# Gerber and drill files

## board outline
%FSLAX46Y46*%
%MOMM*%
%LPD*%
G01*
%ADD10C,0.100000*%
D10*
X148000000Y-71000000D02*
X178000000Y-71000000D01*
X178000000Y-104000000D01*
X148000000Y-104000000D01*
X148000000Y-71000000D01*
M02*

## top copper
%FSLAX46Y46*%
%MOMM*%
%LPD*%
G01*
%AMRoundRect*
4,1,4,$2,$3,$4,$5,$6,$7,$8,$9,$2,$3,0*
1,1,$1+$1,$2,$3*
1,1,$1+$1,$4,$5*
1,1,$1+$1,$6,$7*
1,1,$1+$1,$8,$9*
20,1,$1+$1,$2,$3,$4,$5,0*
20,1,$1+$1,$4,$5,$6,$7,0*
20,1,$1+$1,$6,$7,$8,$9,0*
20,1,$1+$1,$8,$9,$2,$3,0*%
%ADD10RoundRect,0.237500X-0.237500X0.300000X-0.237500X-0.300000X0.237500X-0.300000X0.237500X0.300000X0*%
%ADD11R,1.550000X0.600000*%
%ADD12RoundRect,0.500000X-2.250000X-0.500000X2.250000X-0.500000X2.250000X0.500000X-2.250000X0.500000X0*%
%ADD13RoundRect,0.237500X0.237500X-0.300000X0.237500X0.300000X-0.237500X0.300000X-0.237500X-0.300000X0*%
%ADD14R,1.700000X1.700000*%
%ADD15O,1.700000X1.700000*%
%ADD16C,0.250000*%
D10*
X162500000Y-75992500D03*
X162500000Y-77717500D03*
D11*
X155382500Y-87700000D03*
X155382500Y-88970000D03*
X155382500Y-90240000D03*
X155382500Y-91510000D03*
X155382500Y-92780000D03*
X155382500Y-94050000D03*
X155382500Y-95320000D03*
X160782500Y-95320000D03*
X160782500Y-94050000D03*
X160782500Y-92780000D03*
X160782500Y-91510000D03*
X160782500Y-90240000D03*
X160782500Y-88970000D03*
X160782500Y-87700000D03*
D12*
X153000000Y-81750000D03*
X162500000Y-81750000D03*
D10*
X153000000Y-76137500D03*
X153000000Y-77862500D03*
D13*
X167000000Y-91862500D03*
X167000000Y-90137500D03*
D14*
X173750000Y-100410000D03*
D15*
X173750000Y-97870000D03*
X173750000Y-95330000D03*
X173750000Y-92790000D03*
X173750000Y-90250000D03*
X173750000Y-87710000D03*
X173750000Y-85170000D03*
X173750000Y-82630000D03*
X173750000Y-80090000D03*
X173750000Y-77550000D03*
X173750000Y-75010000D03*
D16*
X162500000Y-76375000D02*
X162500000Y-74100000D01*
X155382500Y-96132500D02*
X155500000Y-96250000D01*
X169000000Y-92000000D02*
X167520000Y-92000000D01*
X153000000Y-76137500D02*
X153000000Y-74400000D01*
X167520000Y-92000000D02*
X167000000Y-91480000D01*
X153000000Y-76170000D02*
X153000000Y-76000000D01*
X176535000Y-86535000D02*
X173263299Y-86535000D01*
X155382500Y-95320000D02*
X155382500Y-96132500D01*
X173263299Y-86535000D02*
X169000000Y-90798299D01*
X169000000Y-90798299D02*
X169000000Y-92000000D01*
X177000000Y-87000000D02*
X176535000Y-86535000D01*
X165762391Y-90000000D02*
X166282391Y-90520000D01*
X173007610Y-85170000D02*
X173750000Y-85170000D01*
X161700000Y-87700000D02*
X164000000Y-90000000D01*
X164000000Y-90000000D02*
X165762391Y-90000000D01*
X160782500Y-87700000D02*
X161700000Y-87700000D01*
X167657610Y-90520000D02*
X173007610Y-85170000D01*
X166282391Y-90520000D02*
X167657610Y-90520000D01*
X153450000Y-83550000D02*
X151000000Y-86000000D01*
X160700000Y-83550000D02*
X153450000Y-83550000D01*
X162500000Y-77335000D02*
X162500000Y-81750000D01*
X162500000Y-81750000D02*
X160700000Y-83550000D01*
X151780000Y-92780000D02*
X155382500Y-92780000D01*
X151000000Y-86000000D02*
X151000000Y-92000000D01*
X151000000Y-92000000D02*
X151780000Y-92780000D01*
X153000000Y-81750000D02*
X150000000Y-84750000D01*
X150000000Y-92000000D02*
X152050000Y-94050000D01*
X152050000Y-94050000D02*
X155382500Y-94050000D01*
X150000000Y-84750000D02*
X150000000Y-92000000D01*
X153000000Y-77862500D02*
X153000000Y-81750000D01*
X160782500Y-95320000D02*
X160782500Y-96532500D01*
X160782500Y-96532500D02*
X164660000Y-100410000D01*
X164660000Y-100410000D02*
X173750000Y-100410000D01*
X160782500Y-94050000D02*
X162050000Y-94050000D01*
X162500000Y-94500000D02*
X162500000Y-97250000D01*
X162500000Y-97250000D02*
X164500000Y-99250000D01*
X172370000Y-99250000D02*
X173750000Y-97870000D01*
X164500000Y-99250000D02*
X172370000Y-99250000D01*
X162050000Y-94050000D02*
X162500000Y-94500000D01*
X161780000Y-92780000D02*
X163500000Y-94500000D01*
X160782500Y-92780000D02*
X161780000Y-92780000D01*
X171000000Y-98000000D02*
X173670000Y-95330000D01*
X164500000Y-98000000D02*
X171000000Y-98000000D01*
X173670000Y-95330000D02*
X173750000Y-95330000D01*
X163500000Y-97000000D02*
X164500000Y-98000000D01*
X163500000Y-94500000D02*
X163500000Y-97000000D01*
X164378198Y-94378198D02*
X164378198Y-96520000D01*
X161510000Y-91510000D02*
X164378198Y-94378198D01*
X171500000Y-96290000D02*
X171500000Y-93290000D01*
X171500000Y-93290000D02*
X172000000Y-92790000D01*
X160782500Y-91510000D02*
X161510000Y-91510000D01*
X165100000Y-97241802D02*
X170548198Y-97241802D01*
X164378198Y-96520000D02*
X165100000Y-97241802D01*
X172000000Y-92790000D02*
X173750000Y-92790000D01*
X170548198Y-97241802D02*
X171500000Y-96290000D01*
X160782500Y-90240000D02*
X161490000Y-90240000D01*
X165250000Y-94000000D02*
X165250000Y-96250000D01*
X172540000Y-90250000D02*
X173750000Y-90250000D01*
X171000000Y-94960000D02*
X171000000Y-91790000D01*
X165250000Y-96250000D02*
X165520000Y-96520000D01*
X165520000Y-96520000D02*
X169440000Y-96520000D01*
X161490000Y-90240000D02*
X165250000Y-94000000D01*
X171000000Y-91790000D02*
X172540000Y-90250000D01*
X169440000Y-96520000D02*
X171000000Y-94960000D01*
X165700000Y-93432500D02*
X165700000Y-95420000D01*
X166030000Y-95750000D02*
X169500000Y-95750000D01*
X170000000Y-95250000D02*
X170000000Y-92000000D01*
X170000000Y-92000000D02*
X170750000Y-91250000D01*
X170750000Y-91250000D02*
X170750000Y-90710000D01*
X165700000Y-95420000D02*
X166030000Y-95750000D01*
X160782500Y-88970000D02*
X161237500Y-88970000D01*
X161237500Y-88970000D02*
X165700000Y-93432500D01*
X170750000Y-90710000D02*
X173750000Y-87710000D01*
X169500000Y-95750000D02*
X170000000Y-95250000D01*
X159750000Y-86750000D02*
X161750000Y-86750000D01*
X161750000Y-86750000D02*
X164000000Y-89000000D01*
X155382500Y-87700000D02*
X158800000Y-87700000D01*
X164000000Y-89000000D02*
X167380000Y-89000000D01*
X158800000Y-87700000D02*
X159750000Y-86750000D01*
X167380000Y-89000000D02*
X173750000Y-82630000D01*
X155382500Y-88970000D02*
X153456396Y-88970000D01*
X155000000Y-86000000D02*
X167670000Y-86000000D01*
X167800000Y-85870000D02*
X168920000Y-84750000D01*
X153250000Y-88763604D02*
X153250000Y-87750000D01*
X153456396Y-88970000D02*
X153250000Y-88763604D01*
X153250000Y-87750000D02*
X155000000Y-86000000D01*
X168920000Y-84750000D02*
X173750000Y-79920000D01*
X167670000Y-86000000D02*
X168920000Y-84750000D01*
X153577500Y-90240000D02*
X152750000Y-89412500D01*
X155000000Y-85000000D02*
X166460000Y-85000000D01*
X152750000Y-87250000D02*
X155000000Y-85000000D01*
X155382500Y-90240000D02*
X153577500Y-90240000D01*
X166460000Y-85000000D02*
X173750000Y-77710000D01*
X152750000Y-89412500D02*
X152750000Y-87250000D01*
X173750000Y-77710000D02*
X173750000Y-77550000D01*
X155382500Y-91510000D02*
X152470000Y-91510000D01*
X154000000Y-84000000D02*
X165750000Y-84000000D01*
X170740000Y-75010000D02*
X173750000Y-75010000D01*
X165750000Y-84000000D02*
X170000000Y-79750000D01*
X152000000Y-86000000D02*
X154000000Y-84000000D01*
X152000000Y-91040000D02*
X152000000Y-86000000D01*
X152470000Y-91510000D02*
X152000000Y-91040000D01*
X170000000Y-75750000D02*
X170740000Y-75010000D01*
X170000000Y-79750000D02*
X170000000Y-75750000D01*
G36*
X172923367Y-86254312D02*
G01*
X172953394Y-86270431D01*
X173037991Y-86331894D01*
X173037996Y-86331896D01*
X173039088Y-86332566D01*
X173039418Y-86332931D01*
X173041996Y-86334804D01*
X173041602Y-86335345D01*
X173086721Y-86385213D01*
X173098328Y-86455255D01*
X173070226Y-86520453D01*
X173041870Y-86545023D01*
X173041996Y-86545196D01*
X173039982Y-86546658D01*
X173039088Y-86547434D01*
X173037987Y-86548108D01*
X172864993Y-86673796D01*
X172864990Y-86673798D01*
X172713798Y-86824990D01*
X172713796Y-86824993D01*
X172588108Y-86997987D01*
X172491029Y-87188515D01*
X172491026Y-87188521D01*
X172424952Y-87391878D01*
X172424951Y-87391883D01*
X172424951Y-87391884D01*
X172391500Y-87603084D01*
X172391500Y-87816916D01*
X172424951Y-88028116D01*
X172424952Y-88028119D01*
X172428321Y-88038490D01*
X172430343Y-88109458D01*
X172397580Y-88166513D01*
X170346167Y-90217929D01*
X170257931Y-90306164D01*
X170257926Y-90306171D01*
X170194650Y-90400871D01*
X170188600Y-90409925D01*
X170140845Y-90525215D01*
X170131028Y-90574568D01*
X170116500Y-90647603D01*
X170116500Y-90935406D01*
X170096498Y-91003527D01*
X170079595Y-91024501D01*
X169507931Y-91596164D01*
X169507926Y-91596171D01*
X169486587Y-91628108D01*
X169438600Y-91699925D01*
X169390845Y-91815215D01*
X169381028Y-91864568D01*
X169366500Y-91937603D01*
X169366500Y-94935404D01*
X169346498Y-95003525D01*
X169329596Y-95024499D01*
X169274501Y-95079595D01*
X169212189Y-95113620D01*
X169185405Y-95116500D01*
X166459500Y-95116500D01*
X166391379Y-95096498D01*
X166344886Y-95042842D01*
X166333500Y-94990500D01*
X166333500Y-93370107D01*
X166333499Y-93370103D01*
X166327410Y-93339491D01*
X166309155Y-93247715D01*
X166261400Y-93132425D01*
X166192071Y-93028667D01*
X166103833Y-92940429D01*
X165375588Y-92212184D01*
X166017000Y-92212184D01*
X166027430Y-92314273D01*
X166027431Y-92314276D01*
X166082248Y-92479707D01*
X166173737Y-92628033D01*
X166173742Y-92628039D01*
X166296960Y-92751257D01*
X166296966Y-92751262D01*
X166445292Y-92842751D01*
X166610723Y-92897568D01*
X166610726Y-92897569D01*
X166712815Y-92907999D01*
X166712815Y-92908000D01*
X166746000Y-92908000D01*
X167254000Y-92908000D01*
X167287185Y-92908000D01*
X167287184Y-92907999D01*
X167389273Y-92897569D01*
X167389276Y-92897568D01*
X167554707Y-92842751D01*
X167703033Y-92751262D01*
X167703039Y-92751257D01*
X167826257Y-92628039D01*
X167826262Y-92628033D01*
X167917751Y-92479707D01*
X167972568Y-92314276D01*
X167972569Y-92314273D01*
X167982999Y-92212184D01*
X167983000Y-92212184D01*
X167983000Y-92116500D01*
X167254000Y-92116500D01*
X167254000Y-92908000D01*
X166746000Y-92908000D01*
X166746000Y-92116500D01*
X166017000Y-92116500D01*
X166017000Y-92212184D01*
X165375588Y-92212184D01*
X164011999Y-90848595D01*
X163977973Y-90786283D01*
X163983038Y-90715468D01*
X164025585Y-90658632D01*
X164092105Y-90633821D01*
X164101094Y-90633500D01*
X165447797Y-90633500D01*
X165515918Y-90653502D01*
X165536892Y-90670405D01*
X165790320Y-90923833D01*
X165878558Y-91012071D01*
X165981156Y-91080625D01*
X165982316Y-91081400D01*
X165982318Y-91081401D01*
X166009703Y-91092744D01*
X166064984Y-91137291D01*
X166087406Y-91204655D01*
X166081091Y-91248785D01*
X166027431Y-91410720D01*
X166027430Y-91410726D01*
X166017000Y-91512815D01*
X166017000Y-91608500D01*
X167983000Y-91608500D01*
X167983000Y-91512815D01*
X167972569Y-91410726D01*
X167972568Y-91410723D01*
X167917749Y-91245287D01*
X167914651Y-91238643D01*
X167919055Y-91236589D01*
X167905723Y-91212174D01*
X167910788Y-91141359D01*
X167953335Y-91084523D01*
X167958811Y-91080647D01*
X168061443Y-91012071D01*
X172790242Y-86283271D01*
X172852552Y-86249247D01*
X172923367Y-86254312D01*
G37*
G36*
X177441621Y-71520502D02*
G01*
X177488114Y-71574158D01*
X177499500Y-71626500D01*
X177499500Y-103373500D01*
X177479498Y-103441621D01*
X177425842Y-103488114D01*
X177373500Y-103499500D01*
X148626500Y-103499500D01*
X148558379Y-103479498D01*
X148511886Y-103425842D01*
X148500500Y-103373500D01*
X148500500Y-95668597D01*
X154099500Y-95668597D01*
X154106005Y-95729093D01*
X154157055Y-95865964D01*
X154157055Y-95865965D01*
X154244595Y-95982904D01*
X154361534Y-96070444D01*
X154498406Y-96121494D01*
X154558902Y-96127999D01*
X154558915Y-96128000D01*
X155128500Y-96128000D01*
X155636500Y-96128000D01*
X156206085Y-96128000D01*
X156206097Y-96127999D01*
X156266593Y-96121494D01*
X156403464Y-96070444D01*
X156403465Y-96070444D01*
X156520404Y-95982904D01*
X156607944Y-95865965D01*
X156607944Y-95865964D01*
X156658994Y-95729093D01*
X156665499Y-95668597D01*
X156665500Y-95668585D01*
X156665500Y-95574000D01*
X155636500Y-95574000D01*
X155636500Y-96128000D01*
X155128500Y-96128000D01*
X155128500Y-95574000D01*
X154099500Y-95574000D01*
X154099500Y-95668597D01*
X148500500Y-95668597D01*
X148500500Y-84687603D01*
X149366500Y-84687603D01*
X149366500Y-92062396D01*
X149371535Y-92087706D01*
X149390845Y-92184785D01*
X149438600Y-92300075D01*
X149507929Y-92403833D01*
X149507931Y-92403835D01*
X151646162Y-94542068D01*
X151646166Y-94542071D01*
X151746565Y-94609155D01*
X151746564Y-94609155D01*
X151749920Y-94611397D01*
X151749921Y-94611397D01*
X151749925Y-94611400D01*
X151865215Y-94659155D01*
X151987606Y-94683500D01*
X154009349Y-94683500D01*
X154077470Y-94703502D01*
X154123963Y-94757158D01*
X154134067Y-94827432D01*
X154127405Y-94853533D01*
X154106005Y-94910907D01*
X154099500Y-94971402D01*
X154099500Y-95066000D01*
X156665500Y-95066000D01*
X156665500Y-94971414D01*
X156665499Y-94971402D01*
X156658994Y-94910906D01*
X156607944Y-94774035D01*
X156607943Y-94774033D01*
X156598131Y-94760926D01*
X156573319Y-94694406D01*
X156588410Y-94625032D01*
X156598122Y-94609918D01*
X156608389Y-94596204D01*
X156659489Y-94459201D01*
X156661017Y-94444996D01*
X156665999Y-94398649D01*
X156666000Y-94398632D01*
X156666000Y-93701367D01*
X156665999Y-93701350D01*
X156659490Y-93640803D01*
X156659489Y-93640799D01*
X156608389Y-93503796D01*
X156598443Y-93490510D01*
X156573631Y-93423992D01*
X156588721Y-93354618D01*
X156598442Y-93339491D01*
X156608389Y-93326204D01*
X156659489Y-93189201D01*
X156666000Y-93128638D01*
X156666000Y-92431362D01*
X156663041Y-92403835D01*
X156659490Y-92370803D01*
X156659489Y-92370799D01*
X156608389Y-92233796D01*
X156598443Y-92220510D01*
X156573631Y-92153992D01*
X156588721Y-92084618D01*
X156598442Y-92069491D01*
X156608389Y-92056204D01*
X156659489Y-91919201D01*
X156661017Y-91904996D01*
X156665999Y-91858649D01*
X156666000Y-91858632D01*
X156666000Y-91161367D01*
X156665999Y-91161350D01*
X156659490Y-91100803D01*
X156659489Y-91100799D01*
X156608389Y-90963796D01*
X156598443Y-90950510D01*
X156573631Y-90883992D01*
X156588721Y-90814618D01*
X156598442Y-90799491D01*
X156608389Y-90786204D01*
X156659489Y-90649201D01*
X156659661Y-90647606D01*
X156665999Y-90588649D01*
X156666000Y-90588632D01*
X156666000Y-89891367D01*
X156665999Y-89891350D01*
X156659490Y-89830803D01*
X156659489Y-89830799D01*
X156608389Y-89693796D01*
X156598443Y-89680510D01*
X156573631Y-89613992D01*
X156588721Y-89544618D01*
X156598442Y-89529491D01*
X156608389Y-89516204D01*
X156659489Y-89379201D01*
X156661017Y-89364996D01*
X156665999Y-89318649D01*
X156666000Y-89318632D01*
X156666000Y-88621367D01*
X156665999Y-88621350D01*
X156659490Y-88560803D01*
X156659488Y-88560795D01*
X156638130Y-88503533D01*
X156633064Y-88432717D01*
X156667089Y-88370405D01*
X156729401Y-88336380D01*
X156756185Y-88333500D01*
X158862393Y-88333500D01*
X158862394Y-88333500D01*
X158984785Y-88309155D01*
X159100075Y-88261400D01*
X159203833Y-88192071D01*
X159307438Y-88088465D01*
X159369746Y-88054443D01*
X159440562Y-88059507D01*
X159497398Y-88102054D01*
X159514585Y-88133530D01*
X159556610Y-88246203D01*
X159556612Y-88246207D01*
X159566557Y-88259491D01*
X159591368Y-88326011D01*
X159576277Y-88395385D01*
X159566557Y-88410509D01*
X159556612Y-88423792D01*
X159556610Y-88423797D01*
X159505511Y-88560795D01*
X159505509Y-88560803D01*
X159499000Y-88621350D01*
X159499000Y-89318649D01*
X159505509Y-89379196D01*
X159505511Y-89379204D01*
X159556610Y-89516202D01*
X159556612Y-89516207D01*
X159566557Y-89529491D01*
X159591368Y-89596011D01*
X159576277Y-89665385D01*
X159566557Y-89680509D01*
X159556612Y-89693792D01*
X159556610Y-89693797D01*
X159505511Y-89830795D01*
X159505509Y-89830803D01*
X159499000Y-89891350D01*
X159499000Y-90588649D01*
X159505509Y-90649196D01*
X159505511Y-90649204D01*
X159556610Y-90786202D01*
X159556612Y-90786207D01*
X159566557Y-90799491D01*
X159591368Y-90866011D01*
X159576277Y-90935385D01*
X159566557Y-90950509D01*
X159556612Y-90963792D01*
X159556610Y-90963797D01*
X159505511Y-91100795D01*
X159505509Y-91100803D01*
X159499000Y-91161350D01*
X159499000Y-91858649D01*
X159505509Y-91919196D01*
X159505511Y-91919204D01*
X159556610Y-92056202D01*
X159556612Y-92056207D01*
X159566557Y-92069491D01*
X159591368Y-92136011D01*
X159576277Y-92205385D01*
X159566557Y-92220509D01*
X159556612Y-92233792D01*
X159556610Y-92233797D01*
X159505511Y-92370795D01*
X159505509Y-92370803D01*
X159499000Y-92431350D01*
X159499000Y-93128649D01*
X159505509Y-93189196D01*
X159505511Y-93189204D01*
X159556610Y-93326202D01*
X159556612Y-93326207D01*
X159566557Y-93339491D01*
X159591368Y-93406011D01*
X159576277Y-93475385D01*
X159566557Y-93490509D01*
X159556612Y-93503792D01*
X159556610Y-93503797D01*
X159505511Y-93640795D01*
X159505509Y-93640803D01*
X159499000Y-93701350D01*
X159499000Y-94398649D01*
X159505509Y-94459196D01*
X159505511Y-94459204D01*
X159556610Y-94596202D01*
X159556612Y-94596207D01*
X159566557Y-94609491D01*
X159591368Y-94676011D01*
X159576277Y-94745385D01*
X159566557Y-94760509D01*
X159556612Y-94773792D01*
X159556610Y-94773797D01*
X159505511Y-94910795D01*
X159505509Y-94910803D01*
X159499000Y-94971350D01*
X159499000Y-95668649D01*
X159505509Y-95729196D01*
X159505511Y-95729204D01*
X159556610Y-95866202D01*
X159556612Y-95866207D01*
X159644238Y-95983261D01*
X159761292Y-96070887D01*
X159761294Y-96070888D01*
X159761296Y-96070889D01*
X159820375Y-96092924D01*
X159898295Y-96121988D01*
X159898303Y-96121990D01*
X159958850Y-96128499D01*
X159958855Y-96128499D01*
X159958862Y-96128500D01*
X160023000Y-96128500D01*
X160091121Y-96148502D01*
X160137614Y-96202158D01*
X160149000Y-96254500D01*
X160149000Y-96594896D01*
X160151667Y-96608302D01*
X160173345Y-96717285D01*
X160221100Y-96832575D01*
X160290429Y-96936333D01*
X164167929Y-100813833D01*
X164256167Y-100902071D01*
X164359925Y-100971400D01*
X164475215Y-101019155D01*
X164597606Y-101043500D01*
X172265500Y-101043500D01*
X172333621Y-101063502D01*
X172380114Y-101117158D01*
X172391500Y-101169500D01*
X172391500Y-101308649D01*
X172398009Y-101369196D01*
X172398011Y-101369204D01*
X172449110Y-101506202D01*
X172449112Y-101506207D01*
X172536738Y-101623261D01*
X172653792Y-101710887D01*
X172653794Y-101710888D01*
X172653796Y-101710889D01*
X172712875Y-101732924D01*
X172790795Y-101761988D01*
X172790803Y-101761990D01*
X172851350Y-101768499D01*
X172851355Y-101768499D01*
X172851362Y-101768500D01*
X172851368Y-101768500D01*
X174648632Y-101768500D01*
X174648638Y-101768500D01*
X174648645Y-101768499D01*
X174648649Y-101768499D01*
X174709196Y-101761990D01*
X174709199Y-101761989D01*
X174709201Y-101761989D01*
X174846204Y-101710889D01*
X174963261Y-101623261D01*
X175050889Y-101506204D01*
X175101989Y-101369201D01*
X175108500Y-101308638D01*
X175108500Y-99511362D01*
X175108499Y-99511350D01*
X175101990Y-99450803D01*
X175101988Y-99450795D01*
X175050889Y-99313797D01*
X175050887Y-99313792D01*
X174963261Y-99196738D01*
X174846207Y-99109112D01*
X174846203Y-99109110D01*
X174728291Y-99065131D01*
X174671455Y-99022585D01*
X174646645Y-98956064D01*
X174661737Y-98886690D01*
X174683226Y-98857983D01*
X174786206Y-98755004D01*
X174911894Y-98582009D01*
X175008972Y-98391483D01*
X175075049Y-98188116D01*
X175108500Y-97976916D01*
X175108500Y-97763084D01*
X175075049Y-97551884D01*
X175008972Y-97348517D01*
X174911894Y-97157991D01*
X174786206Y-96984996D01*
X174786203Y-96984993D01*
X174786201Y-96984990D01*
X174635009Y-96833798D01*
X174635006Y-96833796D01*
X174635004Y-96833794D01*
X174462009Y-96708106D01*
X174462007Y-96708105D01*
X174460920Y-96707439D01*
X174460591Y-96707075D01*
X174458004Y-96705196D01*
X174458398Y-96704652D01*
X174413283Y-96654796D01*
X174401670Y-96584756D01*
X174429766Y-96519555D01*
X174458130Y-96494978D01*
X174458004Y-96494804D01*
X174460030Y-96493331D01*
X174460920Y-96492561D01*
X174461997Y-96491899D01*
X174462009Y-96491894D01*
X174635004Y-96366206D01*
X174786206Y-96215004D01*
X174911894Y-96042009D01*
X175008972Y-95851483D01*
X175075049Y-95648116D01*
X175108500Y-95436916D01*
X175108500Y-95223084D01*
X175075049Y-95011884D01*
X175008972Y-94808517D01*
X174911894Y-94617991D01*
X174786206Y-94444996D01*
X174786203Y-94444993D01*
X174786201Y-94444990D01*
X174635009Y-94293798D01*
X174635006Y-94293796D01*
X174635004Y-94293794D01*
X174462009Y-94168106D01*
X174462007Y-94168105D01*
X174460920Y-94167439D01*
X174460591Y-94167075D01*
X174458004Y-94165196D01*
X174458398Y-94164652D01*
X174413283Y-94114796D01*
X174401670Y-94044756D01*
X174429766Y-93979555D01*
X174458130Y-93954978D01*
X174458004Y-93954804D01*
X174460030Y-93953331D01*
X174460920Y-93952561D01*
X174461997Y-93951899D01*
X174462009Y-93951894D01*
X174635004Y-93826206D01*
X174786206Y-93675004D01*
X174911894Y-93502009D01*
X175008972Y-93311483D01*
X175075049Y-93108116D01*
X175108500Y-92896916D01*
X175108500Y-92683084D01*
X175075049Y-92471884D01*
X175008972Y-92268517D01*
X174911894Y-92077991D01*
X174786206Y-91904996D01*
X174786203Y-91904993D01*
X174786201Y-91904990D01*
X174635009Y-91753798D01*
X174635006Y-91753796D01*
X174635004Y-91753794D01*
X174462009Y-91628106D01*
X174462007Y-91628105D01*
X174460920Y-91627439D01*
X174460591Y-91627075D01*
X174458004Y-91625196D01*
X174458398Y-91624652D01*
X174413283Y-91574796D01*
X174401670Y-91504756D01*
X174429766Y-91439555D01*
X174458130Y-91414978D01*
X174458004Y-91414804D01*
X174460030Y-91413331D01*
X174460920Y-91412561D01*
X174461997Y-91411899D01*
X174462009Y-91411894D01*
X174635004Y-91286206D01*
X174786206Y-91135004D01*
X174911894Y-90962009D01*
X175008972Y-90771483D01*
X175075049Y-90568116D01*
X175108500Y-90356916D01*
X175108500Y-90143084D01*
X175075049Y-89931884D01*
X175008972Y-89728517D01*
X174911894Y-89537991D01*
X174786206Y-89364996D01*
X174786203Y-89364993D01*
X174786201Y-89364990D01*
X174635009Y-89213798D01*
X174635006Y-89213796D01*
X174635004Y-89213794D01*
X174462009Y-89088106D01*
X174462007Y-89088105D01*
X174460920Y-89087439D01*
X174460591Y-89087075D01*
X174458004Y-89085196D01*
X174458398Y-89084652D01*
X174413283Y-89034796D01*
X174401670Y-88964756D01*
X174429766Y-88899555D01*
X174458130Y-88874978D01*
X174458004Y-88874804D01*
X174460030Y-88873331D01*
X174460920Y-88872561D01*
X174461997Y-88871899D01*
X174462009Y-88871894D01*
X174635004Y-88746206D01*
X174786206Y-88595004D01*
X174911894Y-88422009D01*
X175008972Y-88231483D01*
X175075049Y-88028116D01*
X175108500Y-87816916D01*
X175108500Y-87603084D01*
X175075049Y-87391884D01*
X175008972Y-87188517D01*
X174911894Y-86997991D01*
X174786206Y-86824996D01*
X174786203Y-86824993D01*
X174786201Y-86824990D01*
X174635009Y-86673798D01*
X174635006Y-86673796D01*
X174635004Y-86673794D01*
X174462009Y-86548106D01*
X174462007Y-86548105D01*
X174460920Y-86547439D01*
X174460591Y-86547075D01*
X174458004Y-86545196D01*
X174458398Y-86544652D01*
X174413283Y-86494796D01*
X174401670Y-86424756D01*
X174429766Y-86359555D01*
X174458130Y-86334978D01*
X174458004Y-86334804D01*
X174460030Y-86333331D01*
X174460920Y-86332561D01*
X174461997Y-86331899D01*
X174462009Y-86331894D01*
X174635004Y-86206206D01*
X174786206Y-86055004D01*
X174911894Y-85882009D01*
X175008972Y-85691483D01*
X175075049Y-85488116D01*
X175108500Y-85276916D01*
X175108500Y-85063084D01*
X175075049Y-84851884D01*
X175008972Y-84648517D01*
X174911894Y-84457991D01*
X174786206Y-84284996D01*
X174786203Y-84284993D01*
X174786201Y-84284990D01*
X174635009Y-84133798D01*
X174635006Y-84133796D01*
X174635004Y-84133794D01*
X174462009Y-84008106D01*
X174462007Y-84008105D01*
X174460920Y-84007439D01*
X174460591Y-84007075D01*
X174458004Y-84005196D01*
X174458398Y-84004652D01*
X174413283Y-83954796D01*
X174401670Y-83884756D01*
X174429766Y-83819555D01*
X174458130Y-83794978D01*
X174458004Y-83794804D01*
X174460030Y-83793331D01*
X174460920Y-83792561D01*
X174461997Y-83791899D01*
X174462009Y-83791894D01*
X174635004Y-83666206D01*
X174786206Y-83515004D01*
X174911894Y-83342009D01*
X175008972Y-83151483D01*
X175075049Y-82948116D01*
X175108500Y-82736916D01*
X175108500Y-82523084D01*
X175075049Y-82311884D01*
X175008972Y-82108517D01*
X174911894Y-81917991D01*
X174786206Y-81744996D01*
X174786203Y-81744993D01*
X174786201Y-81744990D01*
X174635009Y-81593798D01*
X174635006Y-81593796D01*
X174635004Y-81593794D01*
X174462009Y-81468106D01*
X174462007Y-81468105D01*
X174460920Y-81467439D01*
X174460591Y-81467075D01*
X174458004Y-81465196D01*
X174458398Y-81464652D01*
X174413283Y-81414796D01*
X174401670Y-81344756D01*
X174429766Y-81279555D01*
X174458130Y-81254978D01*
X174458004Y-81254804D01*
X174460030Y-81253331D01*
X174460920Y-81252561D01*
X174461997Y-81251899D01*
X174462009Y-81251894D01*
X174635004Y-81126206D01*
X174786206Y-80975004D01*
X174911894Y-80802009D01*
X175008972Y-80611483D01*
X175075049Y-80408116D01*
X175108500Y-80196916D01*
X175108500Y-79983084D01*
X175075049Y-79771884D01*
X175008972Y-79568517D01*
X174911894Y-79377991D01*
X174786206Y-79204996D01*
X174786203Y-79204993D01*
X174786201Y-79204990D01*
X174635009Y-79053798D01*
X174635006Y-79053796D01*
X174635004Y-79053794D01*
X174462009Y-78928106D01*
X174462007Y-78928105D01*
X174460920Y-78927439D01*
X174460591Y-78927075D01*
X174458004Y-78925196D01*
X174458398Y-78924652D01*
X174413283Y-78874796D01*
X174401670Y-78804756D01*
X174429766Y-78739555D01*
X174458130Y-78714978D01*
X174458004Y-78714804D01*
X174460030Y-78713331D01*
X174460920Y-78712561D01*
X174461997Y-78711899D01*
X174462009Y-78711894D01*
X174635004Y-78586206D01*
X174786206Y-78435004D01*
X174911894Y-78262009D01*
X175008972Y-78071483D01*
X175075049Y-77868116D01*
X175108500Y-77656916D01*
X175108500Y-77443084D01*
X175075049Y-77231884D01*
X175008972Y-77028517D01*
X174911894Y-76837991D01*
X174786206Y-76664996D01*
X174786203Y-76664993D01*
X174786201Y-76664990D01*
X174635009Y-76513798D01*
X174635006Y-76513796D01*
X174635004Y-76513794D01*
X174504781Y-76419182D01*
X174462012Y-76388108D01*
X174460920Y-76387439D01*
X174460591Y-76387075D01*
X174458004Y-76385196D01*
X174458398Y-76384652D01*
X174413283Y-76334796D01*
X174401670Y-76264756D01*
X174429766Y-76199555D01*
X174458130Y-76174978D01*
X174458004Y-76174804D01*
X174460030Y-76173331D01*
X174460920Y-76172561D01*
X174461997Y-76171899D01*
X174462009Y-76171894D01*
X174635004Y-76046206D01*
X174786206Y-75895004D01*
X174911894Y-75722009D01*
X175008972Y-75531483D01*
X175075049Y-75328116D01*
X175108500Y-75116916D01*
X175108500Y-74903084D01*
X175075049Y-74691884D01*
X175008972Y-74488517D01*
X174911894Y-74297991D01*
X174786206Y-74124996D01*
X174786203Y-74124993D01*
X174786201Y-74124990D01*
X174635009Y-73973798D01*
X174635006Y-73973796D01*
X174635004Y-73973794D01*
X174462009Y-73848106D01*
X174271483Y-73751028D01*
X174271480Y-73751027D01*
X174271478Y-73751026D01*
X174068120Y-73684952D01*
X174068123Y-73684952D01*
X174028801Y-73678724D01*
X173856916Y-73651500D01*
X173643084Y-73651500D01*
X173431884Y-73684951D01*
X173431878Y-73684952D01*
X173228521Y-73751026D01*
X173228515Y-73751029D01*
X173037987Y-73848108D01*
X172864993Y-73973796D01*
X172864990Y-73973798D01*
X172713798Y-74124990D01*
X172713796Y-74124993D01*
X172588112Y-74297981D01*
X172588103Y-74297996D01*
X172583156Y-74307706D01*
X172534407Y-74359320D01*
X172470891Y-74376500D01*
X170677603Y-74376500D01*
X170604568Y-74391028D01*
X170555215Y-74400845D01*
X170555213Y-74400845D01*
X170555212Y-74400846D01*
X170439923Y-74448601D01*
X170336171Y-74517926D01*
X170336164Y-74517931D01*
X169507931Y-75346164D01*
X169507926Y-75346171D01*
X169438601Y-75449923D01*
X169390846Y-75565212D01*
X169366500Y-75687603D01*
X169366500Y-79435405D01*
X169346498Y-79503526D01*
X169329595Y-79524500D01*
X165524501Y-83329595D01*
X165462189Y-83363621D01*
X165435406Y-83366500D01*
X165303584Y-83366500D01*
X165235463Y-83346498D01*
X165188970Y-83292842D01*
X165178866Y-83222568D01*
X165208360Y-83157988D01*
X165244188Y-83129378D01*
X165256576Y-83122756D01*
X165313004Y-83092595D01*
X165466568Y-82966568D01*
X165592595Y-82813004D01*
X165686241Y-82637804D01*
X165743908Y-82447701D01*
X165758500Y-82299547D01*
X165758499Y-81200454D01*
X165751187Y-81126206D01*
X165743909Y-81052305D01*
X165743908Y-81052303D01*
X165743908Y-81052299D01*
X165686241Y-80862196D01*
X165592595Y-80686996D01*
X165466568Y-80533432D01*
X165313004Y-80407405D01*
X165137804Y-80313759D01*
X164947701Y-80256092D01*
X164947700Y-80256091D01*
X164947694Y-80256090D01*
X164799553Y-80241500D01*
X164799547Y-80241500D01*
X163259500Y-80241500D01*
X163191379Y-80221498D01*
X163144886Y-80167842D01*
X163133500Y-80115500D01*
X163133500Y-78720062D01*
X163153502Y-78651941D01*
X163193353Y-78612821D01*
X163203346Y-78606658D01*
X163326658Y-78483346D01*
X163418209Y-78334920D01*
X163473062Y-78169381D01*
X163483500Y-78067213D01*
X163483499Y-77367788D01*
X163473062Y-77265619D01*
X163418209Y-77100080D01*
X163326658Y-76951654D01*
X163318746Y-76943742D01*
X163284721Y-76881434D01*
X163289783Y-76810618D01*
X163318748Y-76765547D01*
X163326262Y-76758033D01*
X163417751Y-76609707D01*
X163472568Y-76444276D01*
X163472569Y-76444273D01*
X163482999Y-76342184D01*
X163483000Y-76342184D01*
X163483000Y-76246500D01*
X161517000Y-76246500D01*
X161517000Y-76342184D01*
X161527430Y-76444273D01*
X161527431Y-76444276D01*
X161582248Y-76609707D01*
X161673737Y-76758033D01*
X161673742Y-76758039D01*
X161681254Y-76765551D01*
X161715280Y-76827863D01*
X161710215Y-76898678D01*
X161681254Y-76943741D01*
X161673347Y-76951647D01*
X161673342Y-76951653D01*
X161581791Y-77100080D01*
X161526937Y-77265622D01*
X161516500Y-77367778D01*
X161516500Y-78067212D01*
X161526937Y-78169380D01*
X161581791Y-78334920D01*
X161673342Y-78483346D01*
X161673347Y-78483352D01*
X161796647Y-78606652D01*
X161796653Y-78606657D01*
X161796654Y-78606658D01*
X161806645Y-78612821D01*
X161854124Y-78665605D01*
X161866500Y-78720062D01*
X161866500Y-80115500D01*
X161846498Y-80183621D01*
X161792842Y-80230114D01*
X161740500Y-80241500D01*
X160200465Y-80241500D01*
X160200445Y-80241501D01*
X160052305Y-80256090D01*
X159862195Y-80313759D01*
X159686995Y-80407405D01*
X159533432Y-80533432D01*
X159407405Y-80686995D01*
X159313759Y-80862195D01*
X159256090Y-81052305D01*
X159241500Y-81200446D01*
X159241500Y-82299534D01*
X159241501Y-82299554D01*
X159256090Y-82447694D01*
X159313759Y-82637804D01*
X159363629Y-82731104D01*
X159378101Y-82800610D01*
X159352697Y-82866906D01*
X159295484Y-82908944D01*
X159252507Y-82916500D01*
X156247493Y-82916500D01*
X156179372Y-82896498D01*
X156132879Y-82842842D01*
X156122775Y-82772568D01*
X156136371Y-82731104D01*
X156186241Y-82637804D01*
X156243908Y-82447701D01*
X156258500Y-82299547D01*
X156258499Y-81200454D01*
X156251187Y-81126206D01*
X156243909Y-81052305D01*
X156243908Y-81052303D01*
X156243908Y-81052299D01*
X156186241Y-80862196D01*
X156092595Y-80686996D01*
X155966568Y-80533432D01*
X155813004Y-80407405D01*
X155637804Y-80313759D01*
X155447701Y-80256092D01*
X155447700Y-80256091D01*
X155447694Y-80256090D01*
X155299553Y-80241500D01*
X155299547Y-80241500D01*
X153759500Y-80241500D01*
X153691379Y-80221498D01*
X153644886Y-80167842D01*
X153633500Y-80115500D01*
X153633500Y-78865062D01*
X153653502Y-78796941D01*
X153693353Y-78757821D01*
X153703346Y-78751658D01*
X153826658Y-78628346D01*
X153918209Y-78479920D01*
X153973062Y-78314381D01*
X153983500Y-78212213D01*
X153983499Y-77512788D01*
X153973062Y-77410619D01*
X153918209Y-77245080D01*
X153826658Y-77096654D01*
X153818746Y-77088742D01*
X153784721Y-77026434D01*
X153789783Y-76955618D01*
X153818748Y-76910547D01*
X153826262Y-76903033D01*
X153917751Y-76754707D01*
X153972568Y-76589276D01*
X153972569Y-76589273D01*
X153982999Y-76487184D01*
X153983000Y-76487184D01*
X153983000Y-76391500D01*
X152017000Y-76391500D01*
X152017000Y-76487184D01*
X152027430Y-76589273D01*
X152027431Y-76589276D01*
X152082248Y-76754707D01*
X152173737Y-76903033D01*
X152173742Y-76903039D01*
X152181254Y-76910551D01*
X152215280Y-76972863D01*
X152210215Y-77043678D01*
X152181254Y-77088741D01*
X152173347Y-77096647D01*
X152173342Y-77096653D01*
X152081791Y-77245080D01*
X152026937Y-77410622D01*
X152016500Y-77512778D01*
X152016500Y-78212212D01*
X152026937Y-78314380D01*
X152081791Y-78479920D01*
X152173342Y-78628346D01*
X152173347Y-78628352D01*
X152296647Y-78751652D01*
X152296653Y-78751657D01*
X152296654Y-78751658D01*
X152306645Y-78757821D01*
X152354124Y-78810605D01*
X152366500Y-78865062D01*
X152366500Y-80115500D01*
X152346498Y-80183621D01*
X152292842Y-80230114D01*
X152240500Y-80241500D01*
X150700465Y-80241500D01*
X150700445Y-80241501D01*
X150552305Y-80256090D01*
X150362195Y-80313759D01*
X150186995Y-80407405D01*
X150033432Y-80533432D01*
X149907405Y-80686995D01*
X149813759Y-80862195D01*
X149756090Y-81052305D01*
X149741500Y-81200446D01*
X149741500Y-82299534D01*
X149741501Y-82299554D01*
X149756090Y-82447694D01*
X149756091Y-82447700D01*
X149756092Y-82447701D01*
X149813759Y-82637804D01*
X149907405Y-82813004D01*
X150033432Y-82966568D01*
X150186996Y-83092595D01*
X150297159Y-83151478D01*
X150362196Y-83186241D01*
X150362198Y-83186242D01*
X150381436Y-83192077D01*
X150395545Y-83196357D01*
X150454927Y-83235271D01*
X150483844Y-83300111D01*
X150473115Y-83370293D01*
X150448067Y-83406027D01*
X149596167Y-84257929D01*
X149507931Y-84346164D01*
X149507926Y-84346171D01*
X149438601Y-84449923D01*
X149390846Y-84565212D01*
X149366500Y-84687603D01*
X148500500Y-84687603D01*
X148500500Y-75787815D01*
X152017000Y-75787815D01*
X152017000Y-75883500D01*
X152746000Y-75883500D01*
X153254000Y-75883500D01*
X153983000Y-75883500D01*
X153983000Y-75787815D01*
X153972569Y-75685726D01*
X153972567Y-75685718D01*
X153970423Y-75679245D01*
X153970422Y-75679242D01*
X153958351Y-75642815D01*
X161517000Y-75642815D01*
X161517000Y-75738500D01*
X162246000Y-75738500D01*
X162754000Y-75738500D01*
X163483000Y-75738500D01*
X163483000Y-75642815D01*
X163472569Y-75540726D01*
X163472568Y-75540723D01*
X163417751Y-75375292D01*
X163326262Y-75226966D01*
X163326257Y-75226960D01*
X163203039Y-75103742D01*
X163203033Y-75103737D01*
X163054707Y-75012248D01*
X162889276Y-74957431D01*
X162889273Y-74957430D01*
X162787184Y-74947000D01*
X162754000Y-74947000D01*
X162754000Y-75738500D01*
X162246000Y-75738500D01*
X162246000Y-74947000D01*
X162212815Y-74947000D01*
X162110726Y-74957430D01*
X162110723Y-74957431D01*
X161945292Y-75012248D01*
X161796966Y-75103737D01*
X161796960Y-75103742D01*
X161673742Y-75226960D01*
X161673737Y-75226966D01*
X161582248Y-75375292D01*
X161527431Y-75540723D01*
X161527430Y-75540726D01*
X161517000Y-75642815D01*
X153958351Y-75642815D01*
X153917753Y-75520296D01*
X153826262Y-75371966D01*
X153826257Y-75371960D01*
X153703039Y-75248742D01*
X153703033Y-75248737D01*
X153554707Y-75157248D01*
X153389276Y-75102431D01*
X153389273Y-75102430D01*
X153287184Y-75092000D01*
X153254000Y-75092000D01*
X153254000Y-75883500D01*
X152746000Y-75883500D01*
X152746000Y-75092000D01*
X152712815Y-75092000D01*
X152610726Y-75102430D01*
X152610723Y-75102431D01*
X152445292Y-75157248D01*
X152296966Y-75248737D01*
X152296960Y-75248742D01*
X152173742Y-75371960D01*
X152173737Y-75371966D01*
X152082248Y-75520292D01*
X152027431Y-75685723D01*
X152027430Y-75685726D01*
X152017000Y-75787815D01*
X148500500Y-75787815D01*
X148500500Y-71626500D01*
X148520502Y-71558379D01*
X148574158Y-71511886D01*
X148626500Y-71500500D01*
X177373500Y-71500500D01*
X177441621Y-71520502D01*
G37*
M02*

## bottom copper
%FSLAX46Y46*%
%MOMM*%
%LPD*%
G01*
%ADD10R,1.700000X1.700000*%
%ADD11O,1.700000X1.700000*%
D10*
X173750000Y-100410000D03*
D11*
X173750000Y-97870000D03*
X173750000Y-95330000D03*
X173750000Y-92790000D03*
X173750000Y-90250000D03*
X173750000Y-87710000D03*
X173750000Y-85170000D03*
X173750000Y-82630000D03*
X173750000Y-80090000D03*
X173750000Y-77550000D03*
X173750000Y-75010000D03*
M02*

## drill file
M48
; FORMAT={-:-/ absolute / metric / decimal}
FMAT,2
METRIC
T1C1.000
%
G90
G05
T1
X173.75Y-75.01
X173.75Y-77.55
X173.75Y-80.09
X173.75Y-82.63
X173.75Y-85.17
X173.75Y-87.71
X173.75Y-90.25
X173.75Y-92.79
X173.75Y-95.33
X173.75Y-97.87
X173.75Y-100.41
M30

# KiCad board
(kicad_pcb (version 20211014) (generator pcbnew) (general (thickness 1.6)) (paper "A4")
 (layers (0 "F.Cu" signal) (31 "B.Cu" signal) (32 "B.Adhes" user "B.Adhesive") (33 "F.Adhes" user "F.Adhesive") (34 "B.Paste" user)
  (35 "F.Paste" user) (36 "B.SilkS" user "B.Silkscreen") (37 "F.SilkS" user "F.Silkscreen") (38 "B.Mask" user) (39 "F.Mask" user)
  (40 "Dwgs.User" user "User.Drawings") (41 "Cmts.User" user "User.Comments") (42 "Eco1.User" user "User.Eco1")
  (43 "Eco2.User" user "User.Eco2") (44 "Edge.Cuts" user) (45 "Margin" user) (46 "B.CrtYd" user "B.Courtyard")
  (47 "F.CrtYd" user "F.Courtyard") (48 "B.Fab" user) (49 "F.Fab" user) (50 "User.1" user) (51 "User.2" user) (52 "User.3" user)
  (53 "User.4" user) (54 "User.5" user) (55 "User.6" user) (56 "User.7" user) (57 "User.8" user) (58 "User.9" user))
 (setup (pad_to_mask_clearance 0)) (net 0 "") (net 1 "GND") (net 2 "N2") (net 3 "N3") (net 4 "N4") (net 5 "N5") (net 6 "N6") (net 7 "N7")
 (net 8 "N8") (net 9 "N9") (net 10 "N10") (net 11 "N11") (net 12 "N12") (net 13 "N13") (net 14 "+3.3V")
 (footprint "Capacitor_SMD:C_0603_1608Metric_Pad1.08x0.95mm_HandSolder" (layer "F.Cu") (at 162.5 76.855 -90)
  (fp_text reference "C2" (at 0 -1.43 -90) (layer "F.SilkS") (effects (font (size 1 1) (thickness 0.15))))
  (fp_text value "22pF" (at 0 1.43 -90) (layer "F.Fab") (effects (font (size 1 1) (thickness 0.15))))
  (pad "1" smd roundrect (at -0.8625 0 270) (size 1.075 0.95) (layers "F.Cu" "F.Paste" "F.Mask") (roundrect_rratio 0.25) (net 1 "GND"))
  (pad "2" smd roundrect (at 0.8625 0 270) (size 1.075 0.95) (layers "F.Cu" "F.Paste" "F.Mask") (roundrect_rratio 0.25) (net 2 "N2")))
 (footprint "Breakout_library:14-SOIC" (layer "F.Cu") (at 165.1825 91.18 -90)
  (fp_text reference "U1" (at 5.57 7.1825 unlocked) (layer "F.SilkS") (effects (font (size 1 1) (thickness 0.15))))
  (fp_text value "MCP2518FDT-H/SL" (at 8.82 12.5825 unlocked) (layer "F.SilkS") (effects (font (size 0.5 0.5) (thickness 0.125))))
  (pad "1" smd rect (at -3.48 9.8 90) (size 0.6 1.55) (layers "F.Cu" "F.Paste" "F.Mask") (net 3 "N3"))
  (pad "2" smd rect (at -2.21 9.8 90) (size 0.6 1.55) (layers "F.Cu" "F.Paste" "F.Mask") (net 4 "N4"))
  (pad "3" smd rect (at -0.94 9.8 90) (size 0.6 1.55) (layers "F.Cu" "F.Paste" "F.Mask") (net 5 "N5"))
  (pad "4" smd rect (at 0.33 9.8 90) (size 0.6 1.55) (layers "F.Cu" "F.Paste" "F.Mask") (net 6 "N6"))
  (pad "5" smd rect (at 1.6 9.8 90) (size 0.6 1.55) (layers "F.Cu" "F.Paste" "F.Mask") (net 2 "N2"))
  (pad "6" smd rect (at 2.87 9.8 90) (size 0.6 1.55) (layers "F.Cu" "F.Paste" "F.Mask") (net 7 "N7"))
  (pad "7" smd rect (at 4.14 9.8 90) (size 0.6 1.55) (layers "F.Cu" "F.Paste" "F.Mask") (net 1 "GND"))
  (pad "8" smd rect (at 4.14 4.4 90) (size 0.6 1.55) (layers "F.Cu" "F.Paste" "F.Mask") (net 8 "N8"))
  (pad "9" smd rect (at 2.87 4.4 90) (size 0.6 1.55) (layers "F.Cu" "F.Paste" "F.Mask") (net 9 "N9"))
  (pad "10" smd rect (at 1.6 4.4 90) (size 0.6 1.55) (layers "F.Cu" "F.Paste" "F.Mask") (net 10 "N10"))
  (pad "11" smd rect (at 0.33 4.4 90) (size 0.6 1.55) (layers "F.Cu" "F.Paste" "F.Mask") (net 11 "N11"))
  (pad "12" smd rect (at -0.94 4.4 90) (size 0.6 1.55) (layers "F.Cu" "F.Paste" "F.Mask") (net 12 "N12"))
  (pad "13" smd rect (at -2.21 4.4 90) (size 0.6 1.55) (layers "F.Cu" "F.Paste" "F.Mask") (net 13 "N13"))
  (pad "14" smd rect (at -3.48 4.4 90) (size 0.6 1.55) (layers "F.Cu" "F.Paste" "F.Mask") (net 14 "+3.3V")))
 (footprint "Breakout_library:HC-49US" (layer "F.Cu") (at 157.75 76.75)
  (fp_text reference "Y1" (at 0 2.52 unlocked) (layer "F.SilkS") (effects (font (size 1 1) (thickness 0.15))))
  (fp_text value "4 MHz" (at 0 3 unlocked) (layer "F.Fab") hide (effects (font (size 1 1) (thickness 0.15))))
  (pad "1" smd roundrect (at -4.75 5) (size 5.5 2) (layers "F.Cu" "F.Paste" "F.Mask") (roundrect_rratio 0.25) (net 7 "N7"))
  (pad "2" smd roundrect (at 4.75 5) (size 5.5 2) (layers "F.Cu" "F.Paste" "F.Mask") (roundrect_rratio 0.25) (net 2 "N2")))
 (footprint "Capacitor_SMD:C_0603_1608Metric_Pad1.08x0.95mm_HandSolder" (layer "F.Cu") (at 153 77 -90)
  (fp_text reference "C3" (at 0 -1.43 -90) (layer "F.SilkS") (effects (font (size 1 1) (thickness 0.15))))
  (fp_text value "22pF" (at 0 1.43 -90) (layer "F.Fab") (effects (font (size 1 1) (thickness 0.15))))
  (pad "1" smd roundrect (at -0.8625 0 270) (size 1.075 0.95) (layers "F.Cu" "F.Paste" "F.Mask") (roundrect_rratio 0.25) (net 1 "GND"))
  (pad "2" smd roundrect (at 0.8625 0 270) (size 1.075 0.95) (layers "F.Cu" "F.Paste" "F.Mask") (roundrect_rratio 0.25) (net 7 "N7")))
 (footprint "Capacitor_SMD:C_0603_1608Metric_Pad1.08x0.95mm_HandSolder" (layer "F.Cu") (at 167 91 90)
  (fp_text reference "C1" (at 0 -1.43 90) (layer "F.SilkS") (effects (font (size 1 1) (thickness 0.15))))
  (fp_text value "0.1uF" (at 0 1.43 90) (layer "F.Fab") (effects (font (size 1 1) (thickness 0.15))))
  (pad "1" smd roundrect (at -0.8625 0 90) (size 1.075 0.95) (layers "F.Cu" "F.Paste" "F.Mask") (roundrect_rratio 0.25) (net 1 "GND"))
  (pad "2" smd roundrect (at 0.8625 0 90) (size 1.075 0.95) (layers "F.Cu" "F.Paste" "F.Mask") (roundrect_rratio 0.25) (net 14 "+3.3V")))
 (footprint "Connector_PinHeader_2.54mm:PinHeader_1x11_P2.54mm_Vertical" (layer "F.Cu") (at 173.75 100.41 180)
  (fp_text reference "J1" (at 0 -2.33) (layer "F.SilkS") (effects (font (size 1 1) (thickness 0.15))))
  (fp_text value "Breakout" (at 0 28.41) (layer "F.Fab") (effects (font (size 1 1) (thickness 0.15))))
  (pad "1" thru_hole rect (at 0 0 180) (size 1.7 1.7) (drill 1) (layers *.Cu *.Mask) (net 8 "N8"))
  (pad "2" thru_hole oval (at 0 2.54 180) (size 1.7 1.7) (drill 1) (layers *.Cu *.Mask) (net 9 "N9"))
  (pad "3" thru_hole oval (at 0 5.08 180) (size 1.7 1.7) (drill 1) (layers *.Cu *.Mask) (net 10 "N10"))
  (pad "4" thru_hole oval (at 0 7.62 180) (size 1.7 1.7) (drill 1) (layers *.Cu *.Mask) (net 11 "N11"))
  (pad "5" thru_hole oval (at 0 10.16 180) (size 1.7 1.7) (drill 1) (layers *.Cu *.Mask) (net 12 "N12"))
  (pad "6" thru_hole oval (at 0 12.7 180) (size 1.7 1.7) (drill 1) (layers *.Cu *.Mask) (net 13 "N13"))
  (pad "7" thru_hole oval (at 0 15.24 180) (size 1.7 1.7) (drill 1) (layers *.Cu *.Mask) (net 14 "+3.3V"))
  (pad "8" thru_hole oval (at 0 17.78 180) (size 1.7 1.7) (drill 1) (layers *.Cu *.Mask) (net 3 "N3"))
  (pad "9" thru_hole oval (at 0 20.32 180) (size 1.7 1.7) (drill 1) (layers *.Cu *.Mask) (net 4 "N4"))
  (pad "10" thru_hole oval (at 0 22.86 180) (size 1.7 1.7) (drill 1) (layers *.Cu *.Mask) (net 5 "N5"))
  (pad "11" thru_hole oval (at 0 25.4 180) (size 1.7 1.7) (drill 1) (layers *.Cu *.Mask) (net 6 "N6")))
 (gr_rect (start 148 71) (end 178 104) (layer "Edge.Cuts") (width 0.1) (fill none))
 (segment (start 162.5 76.375) (end 162.5 74.1) (width 0.25) (layer "F.Cu") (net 1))
 (segment (start 155.3825 96.1325) (end 155.5 96.25) (width 0.25) (layer "F.Cu") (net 1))
 (segment (start 169 92) (end 167.52 92) (width 0.25) (layer "F.Cu") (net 1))
 (segment (start 153 76.1375) (end 153 74.4) (width 0.25) (layer "F.Cu") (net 1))
 (segment (start 167.52 92) (end 167 91.48) (width 0.25) (layer "F.Cu") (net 1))
 (segment (start 153 76.17) (end 153 76) (width 0.25) (layer "F.Cu") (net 1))
 (segment (start 176.535 86.535) (end 173.263299 86.535) (width 0.25) (layer "F.Cu") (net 1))
 (segment (start 155.3825 95.32) (end 155.3825 96.1325) (width 0.25) (layer "F.Cu") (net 1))
 (segment (start 173.263299 86.535) (end 169 90.798299) (width 0.25) (layer "F.Cu") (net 1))
 (segment (start 169 90.798299) (end 169 92) (width 0.25) (layer "F.Cu") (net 1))
 (segment (start 177 87) (end 176.535 86.535) (width 0.25) (layer "F.Cu") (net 1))
 (segment (start 165.762391 90) (end 166.282391 90.52) (width 0.25) (layer "F.Cu") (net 14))
 (segment (start 173.00761 85.17) (end 173.75 85.17) (width 0.25) (layer "F.Cu") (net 14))
 (segment (start 161.7 87.7) (end 164 90) (width 0.25) (layer "F.Cu") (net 14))
 (segment (start 164 90) (end 165.762391 90) (width 0.25) (layer "F.Cu") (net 14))
 (segment (start 160.7825 87.7) (end 161.7 87.7) (width 0.25) (layer "F.Cu") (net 14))
 (segment (start 167.65761 90.52) (end 173.00761 85.17) (width 0.25) (layer "F.Cu") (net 14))
 (segment (start 166.282391 90.52) (end 167.65761 90.52) (width 0.25) (layer "F.Cu") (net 14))
 (segment (start 153.45 83.55) (end 151 86) (width 0.25) (layer "F.Cu") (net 2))
 (segment (start 160.7 83.55) (end 153.45 83.55) (width 0.25) (layer "F.Cu") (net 2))
 (segment (start 162.5 77.335) (end 162.5 81.75) (width 0.25) (layer "F.Cu") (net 2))
 (segment (start 162.5 81.75) (end 160.7 83.55) (width 0.25) (layer "F.Cu") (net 2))
 (segment (start 151.78 92.78) (end 155.3825 92.78) (width 0.25) (layer "F.Cu") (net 2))
 (segment (start 151 86) (end 151 92) (width 0.25) (layer "F.Cu") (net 2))
 (segment (start 151 92) (end 151.78 92.78) (width 0.25) (layer "F.Cu") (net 2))
 (segment (start 153 81.75) (end 150 84.75) (width 0.25) (layer "F.Cu") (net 7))
 (segment (start 150 92) (end 152.05 94.05) (width 0.25) (layer "F.Cu") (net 7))
 (segment (start 152.05 94.05) (end 155.3825 94.05) (width 0.25) (layer "F.Cu") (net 7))
 (segment (start 150 84.75) (end 150 92) (width 0.25) (layer "F.Cu") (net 7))
 (segment (start 153 77.8625) (end 153 81.75) (width 0.25) (layer "F.Cu") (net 7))
 (segment (start 160.7825 95.32) (end 160.7825 96.5325) (width 0.25) (layer "F.Cu") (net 8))
 (segment (start 160.7825 96.5325) (end 164.66 100.41) (width 0.25) (layer "F.Cu") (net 8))
 (segment (start 164.66 100.41) (end 173.75 100.41) (width 0.25) (layer "F.Cu") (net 8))
 (segment (start 160.7825 94.05) (end 162.05 94.05) (width 0.25) (layer "F.Cu") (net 9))
 (segment (start 162.5 94.5) (end 162.5 97.25) (width 0.25) (layer "F.Cu") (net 9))
 (segment (start 162.5 97.25) (end 164.5 99.25) (width 0.25) (layer "F.Cu") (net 9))
 (segment (start 172.37 99.25) (end 173.75 97.87) (width 0.25) (layer "F.Cu") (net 9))
 (segment (start 164.5 99.25) (end 172.37 99.25) (width 0.25) (layer "F.Cu") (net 9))
 (segment (start 162.05 94.05) (end 162.5 94.5) (width 0.25) (layer "F.Cu") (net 9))
 (segment (start 161.78 92.78) (end 163.5 94.5) (width 0.25) (layer "F.Cu") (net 10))
 (segment (start 160.7825 92.78) (end 161.78 92.78) (width 0.25) (layer "F.Cu") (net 10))
 (segment (start 171 98) (end 173.67 95.33) (width 0.25) (layer "F.Cu") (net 10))
 (segment (start 164.5 98) (end 171 98) (width 0.25) (layer "F.Cu") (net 10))
 (segment (start 173.67 95.33) (end 173.75 95.33) (width 0.25) (layer "F.Cu") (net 10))
 (segment (start 163.5 97) (end 164.5 98) (width 0.25) (layer "F.Cu") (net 10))
 (segment (start 163.5 94.5) (end 163.5 97) (width 0.25) (layer "F.Cu") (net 10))
 (segment (start 164.378198 94.378198) (end 164.378198 96.52) (width 0.25) (layer "F.Cu") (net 11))
 (segment (start 161.51 91.51) (end 164.378198 94.378198) (width 0.25) (layer "F.Cu") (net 11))
 (segment (start 171.5 96.29) (end 171.5 93.29) (width 0.25) (layer "F.Cu") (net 11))
 (segment (start 171.5 93.29) (end 172 92.79) (width 0.25) (layer "F.Cu") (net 11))
 (segment (start 160.7825 91.51) (end 161.51 91.51) (width 0.25) (layer "F.Cu") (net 11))
 (segment (start 165.1 97.241802) (end 170.548198 97.241802) (width 0.25) (layer "F.Cu") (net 11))
 (segment (start 164.378198 96.52) (end 165.1 97.241802) (width 0.25) (layer "F.Cu") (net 11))
 (segment (start 172 92.79) (end 173.75 92.79) (width 0.25) (layer "F.Cu") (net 11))
 (segment (start 170.548198 97.241802) (end 171.5 96.29) (width 0.25) (layer "F.Cu") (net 11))
 (segment (start 160.7825 90.24) (end 161.49 90.24) (width 0.25) (layer "F.Cu") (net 12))
 (segment (start 165.25 94) (end 165.25 96.25) (width 0.25) (layer "F.Cu") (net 12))
 (segment (start 172.54 90.25) (end 173.75 90.25) (width 0.25) (layer "F.Cu") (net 12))
 (segment (start 171 94.96) (end 171 91.79) (width 0.25) (layer "F.Cu") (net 12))
 (segment (start 165.25 96.25) (end 165.52 96.52) (width 0.25) (layer "F.Cu") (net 12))
 (segment (start 165.52 96.52) (end 169.44 96.52) (width 0.25) (layer "F.Cu") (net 12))
 (segment (start 161.49 90.24) (end 165.25 94) (width 0.25) (layer "F.Cu") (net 12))
 (segment (start 171 91.79) (end 172.54 90.25) (width 0.25) (layer "F.Cu") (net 12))
 (segment (start 169.44 96.52) (end 171 94.96) (width 0.25) (layer "F.Cu") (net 12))
 (segment (start 165.7 93.4325) (end 165.7 95.42) (width 0.25) (layer "F.Cu") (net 13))
 (segment (start 166.03 95.75) (end 169.5 95.75) (width 0.25) (layer "F.Cu") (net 13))
 (segment (start 170 95.25) (end 170 92) (width 0.25) (layer "F.Cu") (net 13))
 (segment (start 170 92) (end 170.75 91.25) (width 0.25) (layer "F.Cu") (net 13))
 (segment (start 170.75 91.25) (end 170.75 90.71) (width 0.25) (layer "F.Cu") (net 13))
 (segment (start 165.7 95.42) (end 166.03 95.75) (width 0.25) (layer "F.Cu") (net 13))
 (segment (start 160.7825 88.97) (end 161.2375 88.97) (width 0.25) (layer "F.Cu") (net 13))
 (segment (start 161.2375 88.97) (end 165.7 93.4325) (width 0.25) (layer "F.Cu") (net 13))
 (segment (start 170.75 90.71) (end 173.75 87.71) (width 0.25) (layer "F.Cu") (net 13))
 (segment (start 169.5 95.75) (end 170 95.25) (width 0.25) (layer "F.Cu") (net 13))
 (segment (start 159.75 86.75) (end 161.75 86.75) (width 0.25) (layer "F.Cu") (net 3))
 (segment (start 161.75 86.75) (end 164 89) (width 0.25) (layer "F.Cu") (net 3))
 (segment (start 155.3825 87.7) (end 158.8 87.7) (width 0.25) (layer "F.Cu") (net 3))
 (segment (start 164 89) (end 167.38 89) (width 0.25) (layer "F.Cu") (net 3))
 (segment (start 158.8 87.7) (end 159.75 86.75) (width 0.25) (layer "F.Cu") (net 3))
 (segment (start 167.38 89) (end 173.75 82.63) (width 0.25) (layer "F.Cu") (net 3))
 (segment (start 155.3825 88.97) (end 153.456396 88.97) (width 0.25) (layer "F.Cu") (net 4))
 (segment (start 155 86) (end 167.67 86) (width 0.25) (layer "F.Cu") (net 4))
 (segment (start 167.8 85.87) (end 168.92 84.75) (width 0.25) (layer "F.Cu") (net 4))
 (segment (start 153.25 88.763604) (end 153.25 87.75) (width 0.25) (layer "F.Cu") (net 4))
 (segment (start 153.456396 88.97) (end 153.25 88.763604) (width 0.25) (layer "F.Cu") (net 4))
 (segment (start 153.25 87.75) (end 155 86) (width 0.25) (layer "F.Cu") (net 4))
 (segment (start 168.92 84.75) (end 173.75 79.92) (width 0.25) (layer "F.Cu") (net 4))
 (segment (start 167.67 86) (end 168.92 84.75) (width 0.25) (layer "F.Cu") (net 4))
 (segment (start 153.5775 90.24) (end 152.75 89.4125) (width 0.25) (layer "F.Cu") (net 5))
 (segment (start 155 85) (end 166.46 85) (width 0.25) (layer "F.Cu") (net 5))
 (segment (start 152.75 87.25) (end 155 85) (width 0.25) (layer "F.Cu") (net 5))
 (segment (start 155.3825 90.24) (end 153.5775 90.24) (width 0.25) (layer "F.Cu") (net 5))
 (segment (start 166.46 85) (end 173.75 77.71) (width 0.25) (layer "F.Cu") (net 5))
 (segment (start 152.75 89.4125) (end 152.75 87.25) (width 0.25) (layer "F.Cu") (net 5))
 (segment (start 173.75 77.71) (end 173.75 77.55) (width 0.25) (layer "F.Cu") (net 5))
 (segment (start 155.3825 91.51) (end 152.47 91.51) (width 0.25) (layer "F.Cu") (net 6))
 (segment (start 154 84) (end 165.75 84) (width 0.25) (layer "F.Cu") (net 6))
 (segment (start 170.74 75.01) (end 173.75 75.01) (width 0.25) (layer "F.Cu") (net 6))
 (segment (start 165.75 84) (end 170 79.75) (width 0.25) (layer "F.Cu") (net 6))
 (segment (start 152 86) (end 154 84) (width 0.25) (layer "F.Cu") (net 6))
 (segment (start 152 91.04) (end 152 86) (width 0.25) (layer "F.Cu") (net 6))
 (segment (start 152.47 91.51) (end 152 91.04) (width 0.25) (layer "F.Cu") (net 6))
 (segment (start 170 75.75) (end 170.74 75.01) (width 0.25) (layer "F.Cu") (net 6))
 (segment (start 170 79.75) (end 170 75.75) (width 0.25) (layer "F.Cu") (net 6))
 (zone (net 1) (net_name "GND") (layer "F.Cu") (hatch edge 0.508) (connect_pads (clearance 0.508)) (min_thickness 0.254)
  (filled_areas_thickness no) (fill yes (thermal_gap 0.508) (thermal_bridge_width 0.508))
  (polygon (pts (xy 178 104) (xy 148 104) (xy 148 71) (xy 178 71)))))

